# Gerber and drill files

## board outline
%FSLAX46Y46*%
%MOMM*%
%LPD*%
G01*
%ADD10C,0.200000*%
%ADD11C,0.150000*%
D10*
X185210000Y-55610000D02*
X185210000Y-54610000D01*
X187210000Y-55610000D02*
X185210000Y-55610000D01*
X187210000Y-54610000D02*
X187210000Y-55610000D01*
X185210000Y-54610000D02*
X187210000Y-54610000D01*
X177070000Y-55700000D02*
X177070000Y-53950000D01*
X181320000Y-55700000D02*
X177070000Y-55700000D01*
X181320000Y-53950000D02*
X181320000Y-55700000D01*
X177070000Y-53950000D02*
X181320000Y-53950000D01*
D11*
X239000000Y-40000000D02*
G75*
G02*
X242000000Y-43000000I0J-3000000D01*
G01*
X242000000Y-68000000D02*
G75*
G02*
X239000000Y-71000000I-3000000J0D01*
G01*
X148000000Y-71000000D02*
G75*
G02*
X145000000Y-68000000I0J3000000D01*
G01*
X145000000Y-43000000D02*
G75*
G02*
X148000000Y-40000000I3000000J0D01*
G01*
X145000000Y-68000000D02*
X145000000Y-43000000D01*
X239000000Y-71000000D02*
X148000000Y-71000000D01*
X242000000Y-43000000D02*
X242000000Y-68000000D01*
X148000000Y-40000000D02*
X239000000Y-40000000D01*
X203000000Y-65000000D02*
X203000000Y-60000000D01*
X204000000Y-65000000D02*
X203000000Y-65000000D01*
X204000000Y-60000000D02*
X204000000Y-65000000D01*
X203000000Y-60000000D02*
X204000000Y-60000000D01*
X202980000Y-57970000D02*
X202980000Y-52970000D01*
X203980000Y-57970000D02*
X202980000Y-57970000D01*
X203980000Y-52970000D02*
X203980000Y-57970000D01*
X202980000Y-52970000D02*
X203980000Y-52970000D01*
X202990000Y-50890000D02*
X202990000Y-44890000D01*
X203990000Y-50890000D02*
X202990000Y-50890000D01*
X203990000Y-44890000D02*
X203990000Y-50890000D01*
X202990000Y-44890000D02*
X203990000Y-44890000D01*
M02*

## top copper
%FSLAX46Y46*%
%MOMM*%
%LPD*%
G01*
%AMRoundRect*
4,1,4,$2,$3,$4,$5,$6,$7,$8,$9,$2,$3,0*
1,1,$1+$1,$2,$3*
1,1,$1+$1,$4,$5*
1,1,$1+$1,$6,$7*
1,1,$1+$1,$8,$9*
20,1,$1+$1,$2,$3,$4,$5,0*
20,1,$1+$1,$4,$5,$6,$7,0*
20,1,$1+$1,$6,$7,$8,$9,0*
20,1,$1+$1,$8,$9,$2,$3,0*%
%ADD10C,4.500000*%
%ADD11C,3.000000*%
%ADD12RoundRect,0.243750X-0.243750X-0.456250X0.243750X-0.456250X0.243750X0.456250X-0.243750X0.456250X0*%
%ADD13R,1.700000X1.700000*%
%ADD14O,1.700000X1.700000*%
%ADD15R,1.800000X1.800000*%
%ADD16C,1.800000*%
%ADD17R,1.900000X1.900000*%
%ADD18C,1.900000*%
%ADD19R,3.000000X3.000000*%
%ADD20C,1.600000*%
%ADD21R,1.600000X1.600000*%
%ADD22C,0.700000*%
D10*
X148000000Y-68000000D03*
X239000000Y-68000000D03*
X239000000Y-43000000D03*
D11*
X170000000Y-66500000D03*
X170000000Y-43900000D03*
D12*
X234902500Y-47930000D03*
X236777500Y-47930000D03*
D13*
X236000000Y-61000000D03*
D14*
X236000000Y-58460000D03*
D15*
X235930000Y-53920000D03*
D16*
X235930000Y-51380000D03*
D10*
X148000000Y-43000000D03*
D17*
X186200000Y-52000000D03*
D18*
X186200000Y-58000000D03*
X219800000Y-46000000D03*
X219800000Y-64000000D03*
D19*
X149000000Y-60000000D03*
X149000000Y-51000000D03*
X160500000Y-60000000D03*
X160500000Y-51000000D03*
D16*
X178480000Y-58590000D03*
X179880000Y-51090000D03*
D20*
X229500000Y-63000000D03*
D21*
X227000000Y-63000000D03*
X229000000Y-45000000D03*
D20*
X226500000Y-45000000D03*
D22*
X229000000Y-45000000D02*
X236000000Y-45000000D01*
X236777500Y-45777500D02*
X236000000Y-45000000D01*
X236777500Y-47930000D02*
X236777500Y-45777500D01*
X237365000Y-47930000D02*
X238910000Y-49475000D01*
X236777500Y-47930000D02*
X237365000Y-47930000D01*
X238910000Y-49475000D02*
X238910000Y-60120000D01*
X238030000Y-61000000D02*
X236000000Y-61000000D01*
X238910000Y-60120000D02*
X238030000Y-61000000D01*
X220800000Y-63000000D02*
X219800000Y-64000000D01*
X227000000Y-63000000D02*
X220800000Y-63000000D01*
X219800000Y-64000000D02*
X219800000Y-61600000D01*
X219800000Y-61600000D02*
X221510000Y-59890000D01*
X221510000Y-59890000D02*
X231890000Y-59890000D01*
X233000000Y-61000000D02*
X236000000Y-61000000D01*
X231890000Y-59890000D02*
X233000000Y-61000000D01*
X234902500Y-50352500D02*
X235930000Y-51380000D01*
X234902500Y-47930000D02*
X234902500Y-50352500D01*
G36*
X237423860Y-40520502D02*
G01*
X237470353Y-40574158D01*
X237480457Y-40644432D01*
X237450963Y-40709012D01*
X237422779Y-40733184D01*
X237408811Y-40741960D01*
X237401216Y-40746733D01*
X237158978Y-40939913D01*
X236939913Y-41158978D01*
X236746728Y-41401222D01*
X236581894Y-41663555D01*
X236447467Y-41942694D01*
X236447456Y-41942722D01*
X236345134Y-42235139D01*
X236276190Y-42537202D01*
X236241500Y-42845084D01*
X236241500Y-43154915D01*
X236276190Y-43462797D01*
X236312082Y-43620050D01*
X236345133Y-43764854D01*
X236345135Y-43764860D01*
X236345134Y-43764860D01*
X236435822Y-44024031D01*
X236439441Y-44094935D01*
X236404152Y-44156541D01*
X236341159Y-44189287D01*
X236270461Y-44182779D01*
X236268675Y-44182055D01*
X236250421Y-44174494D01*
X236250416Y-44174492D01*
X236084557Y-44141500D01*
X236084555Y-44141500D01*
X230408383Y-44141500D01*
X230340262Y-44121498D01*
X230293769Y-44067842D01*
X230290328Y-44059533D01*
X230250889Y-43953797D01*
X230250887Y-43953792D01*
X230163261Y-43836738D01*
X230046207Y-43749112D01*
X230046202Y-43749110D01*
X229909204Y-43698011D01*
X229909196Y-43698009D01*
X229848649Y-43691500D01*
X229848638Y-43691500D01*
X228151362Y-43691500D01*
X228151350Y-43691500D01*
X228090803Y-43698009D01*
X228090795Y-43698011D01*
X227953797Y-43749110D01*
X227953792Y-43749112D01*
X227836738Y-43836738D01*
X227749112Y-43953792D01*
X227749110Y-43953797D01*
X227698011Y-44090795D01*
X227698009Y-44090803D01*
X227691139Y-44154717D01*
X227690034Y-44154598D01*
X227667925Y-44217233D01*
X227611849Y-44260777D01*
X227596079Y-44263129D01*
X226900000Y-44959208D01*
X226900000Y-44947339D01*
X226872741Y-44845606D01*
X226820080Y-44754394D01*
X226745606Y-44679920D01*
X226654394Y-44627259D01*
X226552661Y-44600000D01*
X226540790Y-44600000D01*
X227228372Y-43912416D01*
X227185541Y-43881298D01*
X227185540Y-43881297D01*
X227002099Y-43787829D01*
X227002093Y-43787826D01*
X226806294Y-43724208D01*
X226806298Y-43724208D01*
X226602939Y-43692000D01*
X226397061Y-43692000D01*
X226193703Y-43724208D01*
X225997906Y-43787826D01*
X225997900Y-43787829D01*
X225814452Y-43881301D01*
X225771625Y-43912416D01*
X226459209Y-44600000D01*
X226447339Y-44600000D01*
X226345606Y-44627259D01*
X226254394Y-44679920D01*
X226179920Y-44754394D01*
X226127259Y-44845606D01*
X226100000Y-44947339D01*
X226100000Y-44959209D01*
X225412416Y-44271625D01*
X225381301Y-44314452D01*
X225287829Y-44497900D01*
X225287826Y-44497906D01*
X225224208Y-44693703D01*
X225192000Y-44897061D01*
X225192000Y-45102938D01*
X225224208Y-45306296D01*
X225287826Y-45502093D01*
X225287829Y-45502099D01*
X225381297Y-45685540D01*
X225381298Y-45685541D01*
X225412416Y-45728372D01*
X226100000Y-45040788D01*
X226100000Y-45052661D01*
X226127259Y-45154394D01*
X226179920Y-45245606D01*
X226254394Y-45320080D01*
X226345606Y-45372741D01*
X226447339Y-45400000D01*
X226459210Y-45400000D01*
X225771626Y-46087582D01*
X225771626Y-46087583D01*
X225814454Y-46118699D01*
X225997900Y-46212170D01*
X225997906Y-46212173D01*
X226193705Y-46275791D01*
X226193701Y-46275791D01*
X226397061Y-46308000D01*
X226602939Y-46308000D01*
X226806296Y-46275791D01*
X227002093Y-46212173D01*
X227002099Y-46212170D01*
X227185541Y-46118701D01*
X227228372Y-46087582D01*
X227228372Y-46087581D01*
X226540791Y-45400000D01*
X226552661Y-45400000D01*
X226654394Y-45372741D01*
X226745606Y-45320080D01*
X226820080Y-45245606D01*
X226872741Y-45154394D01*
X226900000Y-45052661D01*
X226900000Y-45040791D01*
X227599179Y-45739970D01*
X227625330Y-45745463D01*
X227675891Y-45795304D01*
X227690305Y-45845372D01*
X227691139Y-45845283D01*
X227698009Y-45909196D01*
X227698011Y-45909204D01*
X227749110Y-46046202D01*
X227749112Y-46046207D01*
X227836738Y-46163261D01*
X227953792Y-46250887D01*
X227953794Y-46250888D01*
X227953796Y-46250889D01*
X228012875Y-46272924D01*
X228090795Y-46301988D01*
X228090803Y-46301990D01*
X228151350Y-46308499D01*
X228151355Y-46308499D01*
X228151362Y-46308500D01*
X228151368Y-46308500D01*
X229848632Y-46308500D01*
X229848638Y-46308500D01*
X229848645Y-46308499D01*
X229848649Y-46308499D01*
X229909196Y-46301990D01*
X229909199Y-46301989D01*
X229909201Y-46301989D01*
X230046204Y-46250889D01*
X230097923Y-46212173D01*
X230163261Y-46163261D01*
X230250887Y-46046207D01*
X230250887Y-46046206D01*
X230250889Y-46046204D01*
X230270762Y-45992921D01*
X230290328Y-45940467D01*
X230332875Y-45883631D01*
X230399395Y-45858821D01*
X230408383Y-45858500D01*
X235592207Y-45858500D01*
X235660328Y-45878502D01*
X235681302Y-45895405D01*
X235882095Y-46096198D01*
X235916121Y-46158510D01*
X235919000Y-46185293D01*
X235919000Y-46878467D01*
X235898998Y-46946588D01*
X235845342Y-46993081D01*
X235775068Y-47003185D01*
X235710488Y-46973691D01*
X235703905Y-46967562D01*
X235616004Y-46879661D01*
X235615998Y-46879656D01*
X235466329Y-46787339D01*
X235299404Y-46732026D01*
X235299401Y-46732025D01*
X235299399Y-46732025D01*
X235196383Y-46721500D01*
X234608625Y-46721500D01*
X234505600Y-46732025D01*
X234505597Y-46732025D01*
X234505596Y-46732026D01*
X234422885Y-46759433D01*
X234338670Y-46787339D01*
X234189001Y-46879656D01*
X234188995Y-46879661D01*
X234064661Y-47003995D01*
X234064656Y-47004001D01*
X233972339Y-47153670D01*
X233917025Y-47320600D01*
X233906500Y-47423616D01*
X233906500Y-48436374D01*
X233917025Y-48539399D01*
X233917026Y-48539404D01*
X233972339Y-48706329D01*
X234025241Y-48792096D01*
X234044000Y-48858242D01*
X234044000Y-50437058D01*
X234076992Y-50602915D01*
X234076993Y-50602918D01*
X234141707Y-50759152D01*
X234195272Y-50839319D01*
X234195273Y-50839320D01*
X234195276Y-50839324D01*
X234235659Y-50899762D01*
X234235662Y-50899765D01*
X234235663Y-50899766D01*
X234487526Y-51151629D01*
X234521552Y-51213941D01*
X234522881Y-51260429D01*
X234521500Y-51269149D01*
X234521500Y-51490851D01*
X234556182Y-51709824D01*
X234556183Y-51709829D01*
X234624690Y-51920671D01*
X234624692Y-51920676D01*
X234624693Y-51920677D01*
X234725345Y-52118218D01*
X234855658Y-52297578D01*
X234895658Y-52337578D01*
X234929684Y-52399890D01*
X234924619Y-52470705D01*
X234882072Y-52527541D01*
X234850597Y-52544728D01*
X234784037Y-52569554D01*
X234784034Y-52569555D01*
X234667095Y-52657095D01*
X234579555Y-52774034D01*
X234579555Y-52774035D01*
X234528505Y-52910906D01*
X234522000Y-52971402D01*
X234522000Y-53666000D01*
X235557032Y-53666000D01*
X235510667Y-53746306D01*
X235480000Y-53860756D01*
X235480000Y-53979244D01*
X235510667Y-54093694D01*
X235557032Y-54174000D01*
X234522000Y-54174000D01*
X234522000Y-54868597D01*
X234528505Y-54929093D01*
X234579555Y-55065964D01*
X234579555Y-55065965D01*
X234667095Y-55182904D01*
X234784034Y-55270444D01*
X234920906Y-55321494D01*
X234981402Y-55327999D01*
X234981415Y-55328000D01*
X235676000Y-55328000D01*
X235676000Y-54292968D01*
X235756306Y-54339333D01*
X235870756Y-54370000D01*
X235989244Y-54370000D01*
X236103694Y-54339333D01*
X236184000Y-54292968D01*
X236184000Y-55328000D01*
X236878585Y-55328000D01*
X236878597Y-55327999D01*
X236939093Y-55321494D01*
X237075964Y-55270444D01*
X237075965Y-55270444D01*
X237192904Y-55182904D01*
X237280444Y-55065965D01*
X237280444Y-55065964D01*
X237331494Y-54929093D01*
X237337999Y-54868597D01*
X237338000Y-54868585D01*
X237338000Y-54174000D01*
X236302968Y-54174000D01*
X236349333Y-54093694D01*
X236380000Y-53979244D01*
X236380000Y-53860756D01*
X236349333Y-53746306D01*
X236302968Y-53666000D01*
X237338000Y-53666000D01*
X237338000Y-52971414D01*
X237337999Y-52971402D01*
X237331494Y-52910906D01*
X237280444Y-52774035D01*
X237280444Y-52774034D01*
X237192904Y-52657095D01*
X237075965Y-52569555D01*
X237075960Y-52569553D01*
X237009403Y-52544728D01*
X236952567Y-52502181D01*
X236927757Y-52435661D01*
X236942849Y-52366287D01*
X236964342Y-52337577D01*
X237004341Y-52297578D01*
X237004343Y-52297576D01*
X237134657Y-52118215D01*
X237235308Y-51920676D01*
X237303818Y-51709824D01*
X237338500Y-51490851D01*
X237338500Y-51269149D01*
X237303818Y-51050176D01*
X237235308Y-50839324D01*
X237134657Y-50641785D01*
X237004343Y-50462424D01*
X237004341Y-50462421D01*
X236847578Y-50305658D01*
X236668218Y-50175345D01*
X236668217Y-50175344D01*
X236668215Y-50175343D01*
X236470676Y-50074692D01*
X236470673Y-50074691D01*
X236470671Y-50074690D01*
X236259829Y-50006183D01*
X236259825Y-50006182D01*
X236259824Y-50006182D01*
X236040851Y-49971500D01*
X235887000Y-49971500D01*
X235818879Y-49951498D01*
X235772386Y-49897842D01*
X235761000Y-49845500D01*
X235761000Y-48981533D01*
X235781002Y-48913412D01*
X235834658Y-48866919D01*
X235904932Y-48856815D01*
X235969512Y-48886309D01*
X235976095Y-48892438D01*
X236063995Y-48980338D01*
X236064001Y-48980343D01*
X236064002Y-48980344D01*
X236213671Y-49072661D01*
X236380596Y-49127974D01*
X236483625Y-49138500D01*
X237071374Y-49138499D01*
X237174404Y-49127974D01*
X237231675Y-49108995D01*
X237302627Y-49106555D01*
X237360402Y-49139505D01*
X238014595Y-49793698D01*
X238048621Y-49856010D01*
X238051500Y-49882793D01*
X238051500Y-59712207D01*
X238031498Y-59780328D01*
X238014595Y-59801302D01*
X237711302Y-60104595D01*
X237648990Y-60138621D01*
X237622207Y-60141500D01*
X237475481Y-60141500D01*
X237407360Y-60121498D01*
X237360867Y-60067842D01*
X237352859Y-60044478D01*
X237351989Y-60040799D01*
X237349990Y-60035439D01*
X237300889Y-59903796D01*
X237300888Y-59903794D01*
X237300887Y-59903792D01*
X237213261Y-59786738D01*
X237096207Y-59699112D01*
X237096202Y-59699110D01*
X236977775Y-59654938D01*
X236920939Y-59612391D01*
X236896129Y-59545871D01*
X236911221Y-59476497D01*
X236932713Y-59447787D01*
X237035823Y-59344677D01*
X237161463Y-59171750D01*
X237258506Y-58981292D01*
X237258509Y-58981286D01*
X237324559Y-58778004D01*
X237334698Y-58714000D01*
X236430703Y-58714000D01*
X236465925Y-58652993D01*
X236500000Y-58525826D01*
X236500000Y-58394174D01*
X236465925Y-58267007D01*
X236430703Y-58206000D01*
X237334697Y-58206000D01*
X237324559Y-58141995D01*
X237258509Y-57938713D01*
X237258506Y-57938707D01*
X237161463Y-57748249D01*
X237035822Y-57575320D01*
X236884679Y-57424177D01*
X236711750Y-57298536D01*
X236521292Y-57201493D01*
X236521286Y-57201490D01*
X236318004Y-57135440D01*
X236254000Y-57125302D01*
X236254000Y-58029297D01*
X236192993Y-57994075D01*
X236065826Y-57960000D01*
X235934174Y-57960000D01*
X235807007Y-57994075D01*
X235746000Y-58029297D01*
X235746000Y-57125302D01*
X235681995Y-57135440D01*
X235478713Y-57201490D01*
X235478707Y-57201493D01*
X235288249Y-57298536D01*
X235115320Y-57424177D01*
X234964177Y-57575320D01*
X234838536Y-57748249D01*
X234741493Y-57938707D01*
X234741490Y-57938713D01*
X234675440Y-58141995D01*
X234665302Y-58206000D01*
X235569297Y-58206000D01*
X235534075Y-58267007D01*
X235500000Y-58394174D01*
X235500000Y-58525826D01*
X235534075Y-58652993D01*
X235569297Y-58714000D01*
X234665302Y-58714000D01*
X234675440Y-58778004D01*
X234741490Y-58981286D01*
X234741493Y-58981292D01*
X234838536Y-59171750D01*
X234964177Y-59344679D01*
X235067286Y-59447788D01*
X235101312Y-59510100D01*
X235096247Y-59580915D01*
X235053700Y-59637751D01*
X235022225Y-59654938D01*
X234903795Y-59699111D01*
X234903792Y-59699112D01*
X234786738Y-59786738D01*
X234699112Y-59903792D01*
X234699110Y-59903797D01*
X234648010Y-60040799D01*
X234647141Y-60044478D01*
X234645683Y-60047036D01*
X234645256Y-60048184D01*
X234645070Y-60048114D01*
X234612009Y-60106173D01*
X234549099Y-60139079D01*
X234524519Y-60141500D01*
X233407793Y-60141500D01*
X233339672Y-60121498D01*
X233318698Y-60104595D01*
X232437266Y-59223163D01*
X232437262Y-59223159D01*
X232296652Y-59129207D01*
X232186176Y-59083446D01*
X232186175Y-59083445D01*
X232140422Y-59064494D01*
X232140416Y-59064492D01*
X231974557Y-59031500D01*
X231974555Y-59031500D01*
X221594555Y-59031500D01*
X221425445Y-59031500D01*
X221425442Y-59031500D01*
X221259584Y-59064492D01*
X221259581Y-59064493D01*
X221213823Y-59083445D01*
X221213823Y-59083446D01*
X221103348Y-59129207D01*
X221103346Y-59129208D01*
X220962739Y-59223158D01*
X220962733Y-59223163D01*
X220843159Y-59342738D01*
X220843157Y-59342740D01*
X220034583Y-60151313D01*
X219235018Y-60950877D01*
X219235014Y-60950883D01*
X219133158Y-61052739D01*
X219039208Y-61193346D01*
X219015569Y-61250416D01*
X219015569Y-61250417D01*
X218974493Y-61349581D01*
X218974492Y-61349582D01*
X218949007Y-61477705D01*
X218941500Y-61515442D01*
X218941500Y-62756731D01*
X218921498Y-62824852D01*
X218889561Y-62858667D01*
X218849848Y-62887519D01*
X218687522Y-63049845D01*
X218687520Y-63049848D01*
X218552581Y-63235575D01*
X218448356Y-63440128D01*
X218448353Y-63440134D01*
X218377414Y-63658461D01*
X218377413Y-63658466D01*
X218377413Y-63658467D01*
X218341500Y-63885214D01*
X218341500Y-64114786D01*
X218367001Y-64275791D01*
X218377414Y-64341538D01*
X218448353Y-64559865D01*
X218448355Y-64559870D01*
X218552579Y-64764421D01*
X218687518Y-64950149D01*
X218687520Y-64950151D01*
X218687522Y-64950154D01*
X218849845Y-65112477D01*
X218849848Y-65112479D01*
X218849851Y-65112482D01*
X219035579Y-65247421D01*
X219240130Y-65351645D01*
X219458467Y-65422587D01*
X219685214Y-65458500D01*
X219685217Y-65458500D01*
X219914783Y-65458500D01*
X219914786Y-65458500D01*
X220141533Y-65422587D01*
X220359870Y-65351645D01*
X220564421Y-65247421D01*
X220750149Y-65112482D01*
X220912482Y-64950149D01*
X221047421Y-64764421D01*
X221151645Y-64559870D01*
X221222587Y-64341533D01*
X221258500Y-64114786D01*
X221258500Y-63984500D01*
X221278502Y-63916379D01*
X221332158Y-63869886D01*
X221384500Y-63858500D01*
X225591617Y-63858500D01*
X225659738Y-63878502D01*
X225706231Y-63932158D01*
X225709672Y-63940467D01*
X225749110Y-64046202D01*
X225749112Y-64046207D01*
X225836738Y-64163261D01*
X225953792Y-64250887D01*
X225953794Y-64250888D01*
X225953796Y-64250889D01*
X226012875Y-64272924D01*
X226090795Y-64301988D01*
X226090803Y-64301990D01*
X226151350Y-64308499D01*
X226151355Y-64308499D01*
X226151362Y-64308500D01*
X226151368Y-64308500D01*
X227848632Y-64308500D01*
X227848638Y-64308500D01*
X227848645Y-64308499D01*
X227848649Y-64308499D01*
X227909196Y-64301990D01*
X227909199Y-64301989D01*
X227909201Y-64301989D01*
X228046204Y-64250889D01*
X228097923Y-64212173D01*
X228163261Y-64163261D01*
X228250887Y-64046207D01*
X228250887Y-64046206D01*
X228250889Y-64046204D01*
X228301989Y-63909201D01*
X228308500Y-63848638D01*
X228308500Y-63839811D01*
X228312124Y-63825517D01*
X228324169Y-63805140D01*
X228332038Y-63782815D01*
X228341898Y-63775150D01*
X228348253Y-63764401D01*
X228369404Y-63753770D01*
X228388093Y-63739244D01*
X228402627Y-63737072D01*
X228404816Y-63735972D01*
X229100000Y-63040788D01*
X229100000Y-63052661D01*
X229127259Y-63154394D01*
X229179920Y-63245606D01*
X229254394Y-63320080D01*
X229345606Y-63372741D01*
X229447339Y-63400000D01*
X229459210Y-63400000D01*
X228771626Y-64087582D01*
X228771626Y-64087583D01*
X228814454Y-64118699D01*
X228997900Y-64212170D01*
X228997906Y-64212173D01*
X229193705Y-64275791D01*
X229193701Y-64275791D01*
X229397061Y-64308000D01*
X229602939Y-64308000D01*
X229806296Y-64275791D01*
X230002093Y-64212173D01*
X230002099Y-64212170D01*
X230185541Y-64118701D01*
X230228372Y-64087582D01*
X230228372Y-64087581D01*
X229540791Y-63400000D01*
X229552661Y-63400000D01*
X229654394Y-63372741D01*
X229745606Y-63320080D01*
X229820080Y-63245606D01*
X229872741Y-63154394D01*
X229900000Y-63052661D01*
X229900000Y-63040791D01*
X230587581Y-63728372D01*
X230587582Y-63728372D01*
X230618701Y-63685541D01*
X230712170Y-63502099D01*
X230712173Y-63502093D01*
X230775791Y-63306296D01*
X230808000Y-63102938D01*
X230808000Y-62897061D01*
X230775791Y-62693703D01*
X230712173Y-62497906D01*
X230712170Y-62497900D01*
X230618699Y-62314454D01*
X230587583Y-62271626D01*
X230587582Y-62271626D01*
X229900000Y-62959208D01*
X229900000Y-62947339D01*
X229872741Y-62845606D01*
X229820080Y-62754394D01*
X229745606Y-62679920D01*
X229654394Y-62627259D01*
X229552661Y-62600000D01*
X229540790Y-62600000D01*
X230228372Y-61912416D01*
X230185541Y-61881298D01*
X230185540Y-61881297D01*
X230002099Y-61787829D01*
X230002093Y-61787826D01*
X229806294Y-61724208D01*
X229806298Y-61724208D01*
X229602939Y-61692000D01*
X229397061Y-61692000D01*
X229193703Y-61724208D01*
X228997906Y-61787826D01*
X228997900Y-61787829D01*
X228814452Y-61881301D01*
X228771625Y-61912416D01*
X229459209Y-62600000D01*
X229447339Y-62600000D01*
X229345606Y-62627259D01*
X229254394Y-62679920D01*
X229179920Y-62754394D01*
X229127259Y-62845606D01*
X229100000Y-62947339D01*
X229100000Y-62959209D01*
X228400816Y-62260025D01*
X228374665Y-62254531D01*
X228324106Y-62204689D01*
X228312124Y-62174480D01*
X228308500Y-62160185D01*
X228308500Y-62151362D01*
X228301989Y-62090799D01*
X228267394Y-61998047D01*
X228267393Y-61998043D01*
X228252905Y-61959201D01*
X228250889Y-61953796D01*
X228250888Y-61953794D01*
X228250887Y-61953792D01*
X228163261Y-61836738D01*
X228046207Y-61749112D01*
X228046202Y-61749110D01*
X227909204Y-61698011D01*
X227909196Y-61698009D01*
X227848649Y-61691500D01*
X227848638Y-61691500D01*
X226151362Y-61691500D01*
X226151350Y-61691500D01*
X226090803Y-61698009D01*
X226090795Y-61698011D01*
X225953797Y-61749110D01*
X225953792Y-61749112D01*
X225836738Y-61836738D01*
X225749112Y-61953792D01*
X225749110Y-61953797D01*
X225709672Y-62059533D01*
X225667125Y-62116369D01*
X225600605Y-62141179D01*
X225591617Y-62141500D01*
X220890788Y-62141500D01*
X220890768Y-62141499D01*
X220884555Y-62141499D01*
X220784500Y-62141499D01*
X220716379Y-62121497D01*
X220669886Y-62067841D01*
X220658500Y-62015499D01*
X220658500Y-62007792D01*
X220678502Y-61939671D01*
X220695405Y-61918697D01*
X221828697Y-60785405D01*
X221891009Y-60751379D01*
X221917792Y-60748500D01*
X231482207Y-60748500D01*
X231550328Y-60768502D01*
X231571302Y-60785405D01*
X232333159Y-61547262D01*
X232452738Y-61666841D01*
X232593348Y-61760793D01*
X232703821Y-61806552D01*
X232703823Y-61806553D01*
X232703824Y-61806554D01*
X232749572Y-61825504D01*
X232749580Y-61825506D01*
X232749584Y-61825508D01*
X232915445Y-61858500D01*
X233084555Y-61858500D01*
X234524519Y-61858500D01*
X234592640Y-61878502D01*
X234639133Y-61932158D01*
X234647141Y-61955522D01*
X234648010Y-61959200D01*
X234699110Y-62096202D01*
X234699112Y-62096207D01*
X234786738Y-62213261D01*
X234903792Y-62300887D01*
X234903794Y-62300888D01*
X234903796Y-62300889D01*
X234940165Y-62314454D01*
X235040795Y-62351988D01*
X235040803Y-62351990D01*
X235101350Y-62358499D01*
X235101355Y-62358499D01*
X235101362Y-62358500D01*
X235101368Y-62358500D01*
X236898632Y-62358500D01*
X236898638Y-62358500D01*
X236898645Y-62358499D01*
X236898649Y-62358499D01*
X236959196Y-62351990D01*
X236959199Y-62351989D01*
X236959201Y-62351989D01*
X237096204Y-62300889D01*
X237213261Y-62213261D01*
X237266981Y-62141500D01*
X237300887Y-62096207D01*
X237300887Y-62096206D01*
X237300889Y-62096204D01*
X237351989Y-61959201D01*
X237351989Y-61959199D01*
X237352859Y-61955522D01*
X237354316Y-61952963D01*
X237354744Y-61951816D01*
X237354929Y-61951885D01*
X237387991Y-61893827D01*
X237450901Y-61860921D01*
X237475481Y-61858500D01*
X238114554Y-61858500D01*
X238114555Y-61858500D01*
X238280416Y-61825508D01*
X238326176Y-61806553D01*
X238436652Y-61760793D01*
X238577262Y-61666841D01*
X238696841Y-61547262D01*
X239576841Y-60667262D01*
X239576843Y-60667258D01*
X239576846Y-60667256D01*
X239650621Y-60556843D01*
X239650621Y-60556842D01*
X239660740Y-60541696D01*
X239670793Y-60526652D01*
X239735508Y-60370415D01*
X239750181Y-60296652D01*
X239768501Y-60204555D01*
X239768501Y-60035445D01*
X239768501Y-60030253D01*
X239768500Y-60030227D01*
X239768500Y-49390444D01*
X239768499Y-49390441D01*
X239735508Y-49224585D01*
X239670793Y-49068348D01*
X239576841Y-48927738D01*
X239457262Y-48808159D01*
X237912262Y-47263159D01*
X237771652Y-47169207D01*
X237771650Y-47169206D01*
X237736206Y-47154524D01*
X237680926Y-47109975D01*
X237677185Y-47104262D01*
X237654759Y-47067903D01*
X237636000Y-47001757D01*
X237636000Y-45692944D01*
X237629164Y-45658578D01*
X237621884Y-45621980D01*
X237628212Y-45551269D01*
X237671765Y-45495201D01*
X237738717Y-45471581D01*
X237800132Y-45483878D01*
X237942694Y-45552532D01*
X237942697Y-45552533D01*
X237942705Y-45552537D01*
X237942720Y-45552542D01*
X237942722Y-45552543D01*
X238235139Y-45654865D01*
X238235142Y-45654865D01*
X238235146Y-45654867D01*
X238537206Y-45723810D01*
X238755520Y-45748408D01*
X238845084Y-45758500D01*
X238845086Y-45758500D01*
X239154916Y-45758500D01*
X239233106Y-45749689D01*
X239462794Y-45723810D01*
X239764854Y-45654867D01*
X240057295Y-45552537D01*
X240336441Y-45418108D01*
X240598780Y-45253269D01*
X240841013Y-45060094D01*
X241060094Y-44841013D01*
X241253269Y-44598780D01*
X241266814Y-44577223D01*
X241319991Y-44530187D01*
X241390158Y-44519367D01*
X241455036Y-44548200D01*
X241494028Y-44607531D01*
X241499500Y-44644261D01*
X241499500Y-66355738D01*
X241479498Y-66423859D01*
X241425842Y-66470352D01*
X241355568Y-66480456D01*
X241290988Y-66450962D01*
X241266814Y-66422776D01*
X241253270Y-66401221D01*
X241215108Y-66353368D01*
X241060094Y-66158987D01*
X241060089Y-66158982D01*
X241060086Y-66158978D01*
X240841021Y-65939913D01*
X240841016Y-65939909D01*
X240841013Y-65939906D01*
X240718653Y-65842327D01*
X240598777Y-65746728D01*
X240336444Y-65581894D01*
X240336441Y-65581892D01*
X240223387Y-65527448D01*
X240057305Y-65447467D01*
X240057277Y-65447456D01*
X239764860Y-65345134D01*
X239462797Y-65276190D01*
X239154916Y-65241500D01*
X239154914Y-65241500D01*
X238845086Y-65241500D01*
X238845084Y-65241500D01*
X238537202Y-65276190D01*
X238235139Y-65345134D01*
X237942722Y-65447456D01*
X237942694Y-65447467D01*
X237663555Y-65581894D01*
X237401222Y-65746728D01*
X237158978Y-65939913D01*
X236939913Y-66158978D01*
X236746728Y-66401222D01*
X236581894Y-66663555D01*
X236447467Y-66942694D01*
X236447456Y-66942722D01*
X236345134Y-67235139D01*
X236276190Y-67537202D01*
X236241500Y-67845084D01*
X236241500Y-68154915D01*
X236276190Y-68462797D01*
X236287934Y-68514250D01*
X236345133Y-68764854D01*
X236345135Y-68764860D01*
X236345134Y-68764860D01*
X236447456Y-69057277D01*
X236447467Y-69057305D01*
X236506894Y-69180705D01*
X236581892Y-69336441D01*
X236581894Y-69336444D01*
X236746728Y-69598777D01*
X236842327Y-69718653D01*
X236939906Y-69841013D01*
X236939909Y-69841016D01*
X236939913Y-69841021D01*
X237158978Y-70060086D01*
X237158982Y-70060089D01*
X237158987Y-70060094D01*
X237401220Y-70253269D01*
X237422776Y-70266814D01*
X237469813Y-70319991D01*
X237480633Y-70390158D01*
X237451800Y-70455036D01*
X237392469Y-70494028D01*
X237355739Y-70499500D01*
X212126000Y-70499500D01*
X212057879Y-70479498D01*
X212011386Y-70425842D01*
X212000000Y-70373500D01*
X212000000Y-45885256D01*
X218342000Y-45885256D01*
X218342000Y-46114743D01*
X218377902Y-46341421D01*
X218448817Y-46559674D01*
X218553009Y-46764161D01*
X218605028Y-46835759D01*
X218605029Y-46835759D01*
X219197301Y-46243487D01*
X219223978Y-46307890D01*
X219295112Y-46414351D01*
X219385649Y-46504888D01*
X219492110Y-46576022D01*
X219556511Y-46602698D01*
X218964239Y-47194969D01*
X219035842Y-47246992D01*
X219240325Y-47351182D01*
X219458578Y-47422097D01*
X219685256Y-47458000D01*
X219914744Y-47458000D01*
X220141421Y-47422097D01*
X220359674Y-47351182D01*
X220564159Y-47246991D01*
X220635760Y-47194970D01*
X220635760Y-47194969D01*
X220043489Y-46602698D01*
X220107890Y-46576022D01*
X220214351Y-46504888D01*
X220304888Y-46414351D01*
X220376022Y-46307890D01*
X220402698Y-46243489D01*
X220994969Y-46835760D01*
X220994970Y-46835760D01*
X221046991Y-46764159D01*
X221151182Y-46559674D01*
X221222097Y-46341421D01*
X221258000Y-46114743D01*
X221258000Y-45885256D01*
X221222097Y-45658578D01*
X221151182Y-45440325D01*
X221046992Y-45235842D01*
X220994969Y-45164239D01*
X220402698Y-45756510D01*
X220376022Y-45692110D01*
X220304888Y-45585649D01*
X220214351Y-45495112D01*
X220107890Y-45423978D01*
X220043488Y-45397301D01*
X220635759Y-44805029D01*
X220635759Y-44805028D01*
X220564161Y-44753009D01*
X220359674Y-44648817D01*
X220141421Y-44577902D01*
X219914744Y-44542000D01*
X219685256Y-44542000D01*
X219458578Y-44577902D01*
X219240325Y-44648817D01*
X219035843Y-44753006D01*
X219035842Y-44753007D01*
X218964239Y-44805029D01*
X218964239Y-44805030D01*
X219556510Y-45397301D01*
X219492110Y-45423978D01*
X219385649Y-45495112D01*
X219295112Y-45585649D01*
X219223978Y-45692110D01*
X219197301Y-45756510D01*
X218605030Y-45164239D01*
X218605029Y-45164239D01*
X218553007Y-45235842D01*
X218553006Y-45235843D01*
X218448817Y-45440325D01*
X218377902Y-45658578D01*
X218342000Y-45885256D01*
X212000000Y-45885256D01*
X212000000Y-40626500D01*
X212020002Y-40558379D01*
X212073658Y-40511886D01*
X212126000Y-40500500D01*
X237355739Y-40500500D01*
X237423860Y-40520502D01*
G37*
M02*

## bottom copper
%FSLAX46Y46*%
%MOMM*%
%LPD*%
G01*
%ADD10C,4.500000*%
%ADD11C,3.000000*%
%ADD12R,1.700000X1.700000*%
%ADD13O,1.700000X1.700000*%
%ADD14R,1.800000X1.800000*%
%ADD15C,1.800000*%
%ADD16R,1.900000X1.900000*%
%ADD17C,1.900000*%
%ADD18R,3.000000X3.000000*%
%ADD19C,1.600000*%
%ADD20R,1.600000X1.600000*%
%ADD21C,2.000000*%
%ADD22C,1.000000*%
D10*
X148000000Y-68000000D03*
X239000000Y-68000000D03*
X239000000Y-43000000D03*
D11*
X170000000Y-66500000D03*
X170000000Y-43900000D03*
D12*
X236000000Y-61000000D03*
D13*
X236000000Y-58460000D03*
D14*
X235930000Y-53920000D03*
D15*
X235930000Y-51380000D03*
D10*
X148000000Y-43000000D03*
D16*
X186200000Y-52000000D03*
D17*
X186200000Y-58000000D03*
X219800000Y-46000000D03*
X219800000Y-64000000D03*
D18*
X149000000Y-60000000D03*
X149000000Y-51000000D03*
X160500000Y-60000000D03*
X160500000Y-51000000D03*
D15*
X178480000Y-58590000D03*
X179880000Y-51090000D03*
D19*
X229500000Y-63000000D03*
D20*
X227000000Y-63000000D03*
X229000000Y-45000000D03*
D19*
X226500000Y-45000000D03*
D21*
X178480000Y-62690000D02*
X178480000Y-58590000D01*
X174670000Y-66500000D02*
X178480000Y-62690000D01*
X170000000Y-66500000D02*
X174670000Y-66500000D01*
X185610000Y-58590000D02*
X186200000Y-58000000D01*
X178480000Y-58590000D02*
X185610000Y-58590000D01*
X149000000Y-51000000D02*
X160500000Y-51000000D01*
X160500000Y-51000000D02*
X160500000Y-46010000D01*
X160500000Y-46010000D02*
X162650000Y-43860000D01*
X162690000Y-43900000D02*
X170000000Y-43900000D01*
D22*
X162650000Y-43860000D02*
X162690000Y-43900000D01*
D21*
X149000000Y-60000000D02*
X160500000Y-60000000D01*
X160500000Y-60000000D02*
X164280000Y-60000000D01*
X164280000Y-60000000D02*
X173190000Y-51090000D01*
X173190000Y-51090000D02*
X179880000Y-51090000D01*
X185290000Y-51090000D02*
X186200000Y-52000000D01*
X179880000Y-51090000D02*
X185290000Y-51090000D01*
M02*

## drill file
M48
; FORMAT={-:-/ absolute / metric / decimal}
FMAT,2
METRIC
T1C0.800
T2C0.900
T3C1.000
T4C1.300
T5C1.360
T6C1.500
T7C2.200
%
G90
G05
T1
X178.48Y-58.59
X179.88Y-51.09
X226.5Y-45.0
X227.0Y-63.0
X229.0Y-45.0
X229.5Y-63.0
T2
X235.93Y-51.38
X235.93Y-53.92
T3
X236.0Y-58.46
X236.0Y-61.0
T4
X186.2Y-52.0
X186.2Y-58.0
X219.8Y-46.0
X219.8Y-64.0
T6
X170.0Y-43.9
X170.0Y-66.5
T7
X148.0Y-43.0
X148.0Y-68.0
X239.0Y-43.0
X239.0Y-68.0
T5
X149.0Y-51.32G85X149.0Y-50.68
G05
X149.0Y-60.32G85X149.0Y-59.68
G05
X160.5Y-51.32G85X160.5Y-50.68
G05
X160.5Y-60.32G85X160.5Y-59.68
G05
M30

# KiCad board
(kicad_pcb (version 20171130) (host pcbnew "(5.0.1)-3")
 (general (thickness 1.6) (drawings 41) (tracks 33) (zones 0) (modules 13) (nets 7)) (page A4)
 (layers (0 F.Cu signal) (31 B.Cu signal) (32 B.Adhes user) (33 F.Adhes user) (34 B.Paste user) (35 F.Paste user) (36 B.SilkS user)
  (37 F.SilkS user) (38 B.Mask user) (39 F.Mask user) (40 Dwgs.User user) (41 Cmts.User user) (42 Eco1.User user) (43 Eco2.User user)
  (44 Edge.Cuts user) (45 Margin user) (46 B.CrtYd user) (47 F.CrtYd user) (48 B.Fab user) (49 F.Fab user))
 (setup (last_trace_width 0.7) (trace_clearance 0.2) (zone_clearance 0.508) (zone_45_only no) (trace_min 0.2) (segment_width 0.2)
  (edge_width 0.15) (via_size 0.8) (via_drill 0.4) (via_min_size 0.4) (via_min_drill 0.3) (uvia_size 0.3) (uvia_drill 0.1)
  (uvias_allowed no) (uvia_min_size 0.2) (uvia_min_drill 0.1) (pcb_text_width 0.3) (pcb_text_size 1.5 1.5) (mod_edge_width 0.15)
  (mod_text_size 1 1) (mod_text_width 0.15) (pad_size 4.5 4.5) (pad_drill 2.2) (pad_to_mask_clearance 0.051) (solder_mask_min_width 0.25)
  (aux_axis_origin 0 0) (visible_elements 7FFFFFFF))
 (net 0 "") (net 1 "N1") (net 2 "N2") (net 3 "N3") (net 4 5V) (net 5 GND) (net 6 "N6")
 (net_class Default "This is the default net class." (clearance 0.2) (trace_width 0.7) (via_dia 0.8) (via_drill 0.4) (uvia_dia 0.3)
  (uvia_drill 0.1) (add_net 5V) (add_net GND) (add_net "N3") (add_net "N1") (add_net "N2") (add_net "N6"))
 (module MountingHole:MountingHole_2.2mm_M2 (layer F.Cu) (at 148 68)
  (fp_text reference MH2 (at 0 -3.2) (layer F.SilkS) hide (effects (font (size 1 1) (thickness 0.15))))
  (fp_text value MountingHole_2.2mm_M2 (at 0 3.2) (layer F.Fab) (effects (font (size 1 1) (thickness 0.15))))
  (pad "" np_thru_hole circle (at 0 0) (size 4.5 4.5) (drill 2.2) (layers *.Cu *.Mask)))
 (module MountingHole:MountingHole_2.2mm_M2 (layer F.Cu) (at 239 68)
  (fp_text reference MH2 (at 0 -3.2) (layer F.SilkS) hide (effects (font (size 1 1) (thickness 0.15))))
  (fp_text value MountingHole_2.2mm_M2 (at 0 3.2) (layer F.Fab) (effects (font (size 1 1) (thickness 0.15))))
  (pad "" np_thru_hole circle (at 0 0) (size 4.5 4.5) (drill 2.2) (layers *.Cu *.Mask)))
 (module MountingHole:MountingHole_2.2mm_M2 (layer F.Cu) (at 239 43)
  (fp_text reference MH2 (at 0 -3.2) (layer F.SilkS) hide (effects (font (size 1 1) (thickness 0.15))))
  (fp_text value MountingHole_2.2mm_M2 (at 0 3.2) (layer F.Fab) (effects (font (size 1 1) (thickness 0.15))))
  (pad "" np_thru_hole circle (at 0 0) (size 4.5 4.5) (drill 2.2) (layers *.Cu *.Mask)))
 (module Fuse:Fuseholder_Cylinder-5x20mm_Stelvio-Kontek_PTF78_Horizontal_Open (layer F.Cu) (at 170 66.5 90)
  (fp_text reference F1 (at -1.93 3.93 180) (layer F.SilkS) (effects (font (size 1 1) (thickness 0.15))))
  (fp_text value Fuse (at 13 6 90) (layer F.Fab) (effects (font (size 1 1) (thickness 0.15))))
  (pad 1 thru_hole circle (at 0 0 90) (size 3 3) (drill 1.5) (layers *.Cu *.Mask) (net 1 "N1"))
  (pad 2 thru_hole circle (at 22.6 0 90) (size 3 3) (drill 1.5) (layers *.Cu *.Mask) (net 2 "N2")))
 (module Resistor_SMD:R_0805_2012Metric (layer F.Cu) (at 235.84 47.93)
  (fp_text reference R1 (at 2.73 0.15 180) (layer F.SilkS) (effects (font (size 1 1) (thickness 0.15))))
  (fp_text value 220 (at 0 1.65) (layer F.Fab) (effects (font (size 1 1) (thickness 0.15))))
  (pad 1 smd roundrect (at -0.9375 0) (size 0.975 1.4) (layers F.Cu F.Paste F.Mask) (roundrect_rratio 0.25) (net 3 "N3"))
  (pad 2 smd roundrect (at 0.9375 0) (size 0.975 1.4) (layers F.Cu F.Paste F.Mask) (roundrect_rratio 0.25) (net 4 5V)))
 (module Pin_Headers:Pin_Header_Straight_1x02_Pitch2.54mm (layer F.Cu) (at 236 61 180)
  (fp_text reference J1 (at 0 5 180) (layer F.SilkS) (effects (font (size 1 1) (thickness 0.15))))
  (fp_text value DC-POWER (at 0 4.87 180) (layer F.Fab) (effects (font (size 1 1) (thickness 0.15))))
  (pad 1 thru_hole rect (at 0 0 180) (size 1.7 1.7) (drill 1) (layers *.Cu *.Mask) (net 4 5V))
  (pad 2 thru_hole oval (at 0 2.54 180) (size 1.7 1.7) (drill 1) (layers *.Cu *.Mask) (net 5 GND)))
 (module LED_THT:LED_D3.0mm (layer F.Cu) (at 235.93 53.92 90)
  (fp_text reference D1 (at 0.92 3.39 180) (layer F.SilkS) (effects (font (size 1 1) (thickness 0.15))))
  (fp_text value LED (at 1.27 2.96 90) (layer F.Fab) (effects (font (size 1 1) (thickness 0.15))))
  (pad 1 thru_hole rect (at 0 0 90) (size 1.8 1.8) (drill 0.9) (layers *.Cu *.Mask) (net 5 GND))
  (pad 2 thru_hole circle (at 2.54 0 90) (size 1.8 1.8) (drill 0.9) (layers *.Cu *.Mask) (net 3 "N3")))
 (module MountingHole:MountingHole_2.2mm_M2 (layer F.Cu) (at 148 43)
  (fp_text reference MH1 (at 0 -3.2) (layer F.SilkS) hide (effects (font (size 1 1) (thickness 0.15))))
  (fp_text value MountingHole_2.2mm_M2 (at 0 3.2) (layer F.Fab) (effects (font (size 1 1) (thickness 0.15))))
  (pad "" np_thru_hole circle (at 0 0) (size 4.5 4.5) (drill 2.2) (layers *.Cu *.Mask)))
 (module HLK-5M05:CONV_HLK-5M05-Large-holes (layer F.Cu) (at 203 55)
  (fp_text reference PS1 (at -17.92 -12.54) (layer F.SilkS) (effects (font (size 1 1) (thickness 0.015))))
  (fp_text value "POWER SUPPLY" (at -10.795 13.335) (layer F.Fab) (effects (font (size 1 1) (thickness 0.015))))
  (pad 1 thru_hole rect (at -16.8 -3) (size 1.9 1.9) (drill 1.3) (layers *.Cu *.Mask) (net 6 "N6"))
  (pad 2 thru_hole circle (at -16.8 3) (size 1.9 1.9) (drill 1.3) (layers *.Cu *.Mask) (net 1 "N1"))
  (pad 3 thru_hole circle (at 16.8 -9) (size 1.9 1.9) (drill 1.3) (layers *.Cu *.Mask) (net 5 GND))
  (pad 4 thru_hole circle (at 16.8 9) (size 1.9 1.9) (drill 1.3) (layers *.Cu *.Mask) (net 4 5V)))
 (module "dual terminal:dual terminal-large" (layer F.Cu) (at 149 60 90)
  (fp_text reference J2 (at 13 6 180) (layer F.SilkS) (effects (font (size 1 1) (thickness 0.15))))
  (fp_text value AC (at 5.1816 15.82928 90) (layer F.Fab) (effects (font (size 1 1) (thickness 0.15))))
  (pad 1 thru_hole rect (at 0 0 90) (size 3 3) (drill oval 2 1.36) (layers *.Cu *.Mask) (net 6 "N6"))
  (pad 2 thru_hole rect (at 9 0 90) (size 3 3) (drill oval 2 1.36) (layers *.Cu *.Mask) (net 2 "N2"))
  (pad 1 thru_hole rect (at 0 11.5 90) (size 3 3) (drill oval 2 1.36) (layers *.Cu *.Mask) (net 6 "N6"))
  (pad 2 thru_hole rect (at 9 11.5 90) (size 3 3) (drill oval 2 1.36) (layers *.Cu *.Mask) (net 2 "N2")))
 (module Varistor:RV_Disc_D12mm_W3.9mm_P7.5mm (layer F.Cu) (at 178.48 58.59 90)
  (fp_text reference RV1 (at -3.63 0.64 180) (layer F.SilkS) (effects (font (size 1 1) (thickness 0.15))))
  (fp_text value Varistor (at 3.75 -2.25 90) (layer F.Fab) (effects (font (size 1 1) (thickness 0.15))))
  (pad 1 thru_hole circle (at 0 0 90) (size 1.8 1.8) (drill 0.8) (layers *.Cu *.Mask) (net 1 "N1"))
  (pad 2 thru_hole circle (at 7.5 1.4 90) (size 1.8 1.8) (drill 0.8) (layers *.Cu *.Mask) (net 6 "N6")))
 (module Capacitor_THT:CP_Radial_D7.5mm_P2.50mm (layer F.Cu) (at 227 63)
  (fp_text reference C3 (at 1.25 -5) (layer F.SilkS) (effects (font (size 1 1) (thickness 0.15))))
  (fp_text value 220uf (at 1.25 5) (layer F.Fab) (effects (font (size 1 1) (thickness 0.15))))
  (pad 2 thru_hole circle (at 2.5 0) (size 1.6 1.6) (drill 0.8) (layers *.Cu *.Mask) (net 5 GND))
  (pad 1 thru_hole rect (at 0 0) (size 1.6 1.6) (drill 0.8) (layers *.Cu *.Mask) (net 4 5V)))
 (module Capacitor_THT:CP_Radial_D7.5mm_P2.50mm (layer F.Cu) (at 229 45 180)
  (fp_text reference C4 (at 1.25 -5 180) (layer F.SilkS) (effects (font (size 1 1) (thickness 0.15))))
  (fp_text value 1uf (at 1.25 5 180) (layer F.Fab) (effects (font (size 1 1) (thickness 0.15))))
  (pad 1 thru_hole rect (at 0 0 180) (size 1.6 1.6) (drill 0.8) (layers *.Cu *.Mask) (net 4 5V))
  (pad 2 thru_hole circle (at 2.5 0 180) (size 1.6 1.6) (drill 0.8) (layers *.Cu *.Mask) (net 5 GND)))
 (gr_line (start 185.21 55.61) (end 185.21 54.61) (layer Edge.Cuts) (width 0.2))
 (gr_line (start 187.21 55.61) (end 185.21 55.61) (layer Edge.Cuts) (width 0.2))
 (gr_line (start 187.21 54.61) (end 187.21 55.61) (layer Edge.Cuts) (width 0.2))
 (gr_line (start 185.21 54.61) (end 187.21 54.61) (layer Edge.Cuts) (width 0.2))
 (gr_line (start 177.07 55.7) (end 177.07 53.95) (layer Edge.Cuts) (width 0.2))
 (gr_line (start 181.32 55.7) (end 177.07 55.7) (layer Edge.Cuts) (width 0.2))
 (gr_line (start 181.32 53.95) (end 181.32 55.7) (layer Edge.Cuts) (width 0.2))
 (gr_line (start 177.07 53.95) (end 181.32 53.95) (layer Edge.Cuts) (width 0.2))
 (gr_arc (start 239 43) (end 242 43) (angle -90) (layer Edge.Cuts) (width 0.15))
 (gr_arc (start 239 68) (end 239 71) (angle -90) (layer Edge.Cuts) (width 0.15))
 (gr_arc (start 148 68) (end 145 68) (angle -90) (layer Edge.Cuts) (width 0.15))
 (gr_arc (start 148 43) (end 148 40) (angle -90) (layer Edge.Cuts) (width 0.15))
 (gr_line (start 145 68) (end 145 43) (layer Edge.Cuts) (width 0.15))
 (gr_line (start 239 71) (end 148 71) (layer Edge.Cuts) (width 0.15))
 (gr_line (start 242 43) (end 242 68) (layer Edge.Cuts) (width 0.15))
 (gr_line (start 148 40) (end 239 40) (layer Edge.Cuts) (width 0.15))
 (gr_line (start 203 65) (end 203 60) (layer Edge.Cuts) (width 0.15))
 (gr_line (start 204 65) (end 203 65) (layer Edge.Cuts) (width 0.15))
 (gr_line (start 204 60) (end 204 65) (layer Edge.Cuts) (width 0.15))
 (gr_line (start 203 60) (end 204 60) (layer Edge.Cuts) (width 0.15))
 (gr_line (start 202.98 57.97) (end 202.98 52.97) (layer Edge.Cuts) (width 0.15))
 (gr_line (start 203.98 57.97) (end 202.98 57.97) (layer Edge.Cuts) (width 0.15))
 (gr_line (start 203.98 52.97) (end 203.98 57.97) (layer Edge.Cuts) (width 0.15))
 (gr_line (start 202.98 52.97) (end 203.98 52.97) (layer Edge.Cuts) (width 0.15))
 (gr_line (start 202.99 50.89) (end 202.99 44.89) (layer Edge.Cuts) (width 0.15))
 (gr_line (start 203.99 50.89) (end 202.99 50.89) (layer Edge.Cuts) (width 0.15))
 (gr_line (start 203.99 44.89) (end 203.99 50.89) (layer Edge.Cuts) (width 0.15))
 (gr_line (start 202.99 44.89) (end 203.99 44.89) (layer Edge.Cuts) (width 0.15))
 (segment (start 178.48 62.69) (end 178.48 58.59) (width 2) (layer B.Cu) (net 1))
 (segment (start 174.67 66.5) (end 178.48 62.69) (width 2) (layer B.Cu) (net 1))
 (segment (start 170 66.5) (end 174.67 66.5) (width 2) (layer B.Cu) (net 1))
 (segment (start 185.61 58.59) (end 186.2 58) (width 2) (layer B.Cu) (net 1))
 (segment (start 178.48 58.59) (end 185.61 58.59) (width 2) (layer B.Cu) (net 1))
 (segment (start 149 51) (end 160.5 51) (width 2) (layer B.Cu) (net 2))
 (segment (start 160.5 51) (end 160.5 46.01) (width 2) (layer B.Cu) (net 2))
 (segment (start 160.5 46.01) (end 162.65 43.86) (width 2) (layer B.Cu) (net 2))
 (segment (start 162.69 43.9) (end 170 43.9) (width 2) (layer B.Cu) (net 2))
 (segment (start 162.65 43.86) (end 162.69 43.9) (width 1) (layer B.Cu) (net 2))
 (segment (start 149 60) (end 160.5 60) (width 2) (layer B.Cu) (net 6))
 (segment (start 160.5 60) (end 164.28 60) (width 2) (layer B.Cu) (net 6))
 (segment (start 164.28 60) (end 173.19 51.09) (width 2) (layer B.Cu) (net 6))
 (segment (start 173.19 51.09) (end 179.88 51.09) (width 2) (layer B.Cu) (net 6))
 (segment (start 185.29 51.09) (end 186.2 52) (width 2) (layer B.Cu) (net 6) (status 1000000))
 (segment (start 179.88 51.09) (end 185.29 51.09) (width 2) (layer B.Cu) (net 6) (status 1000000))
 (segment (start 229 45) (end 236 45) (width 0.7) (layer F.Cu) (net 4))
 (segment (start 236.7775 45.7775) (end 236 45) (width 0.7) (layer F.Cu) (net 4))
 (segment (start 236.7775 47.93) (end 236.7775 45.7775) (width 0.7) (layer F.Cu) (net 4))
 (segment (start 237.365 47.93) (end 238.91 49.475) (width 0.7) (layer F.Cu) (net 4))
 (segment (start 236.7775 47.93) (end 237.365 47.93) (width 0.7) (layer F.Cu) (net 4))
 (segment (start 238.91 49.475) (end 238.91 60.12) (width 0.7) (layer F.Cu) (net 4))
 (segment (start 238.03 61) (end 236 61) (width 0.7) (layer F.Cu) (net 4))
 (segment (start 238.91 60.12) (end 238.03 61) (width 0.7) (layer F.Cu) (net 4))
 (segment (start 220.8 63) (end 219.8 64) (width 0.7) (layer F.Cu) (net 4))
 (segment (start 227 63) (end 220.8 63) (width 0.7) (layer F.Cu) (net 4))
 (segment (start 219.8 64) (end 219.8 61.6) (width 0.7) (layer F.Cu) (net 4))
 (segment (start 219.8 61.6) (end 221.51 59.89) (width 0.7) (layer F.Cu) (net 4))
 (segment (start 221.51 59.89) (end 231.89 59.89) (width 0.7) (layer F.Cu) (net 4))
 (segment (start 233 61) (end 236 61) (width 0.7) (layer F.Cu) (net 4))
 (segment (start 231.89 59.89) (end 233 61) (width 0.7) (layer F.Cu) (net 4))
 (segment (start 234.9025 50.3525) (end 235.93 51.38) (width 0.7) (layer F.Cu) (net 3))
 (segment (start 234.9025 47.93) (end 234.9025 50.3525) (width 0.7) (layer F.Cu) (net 3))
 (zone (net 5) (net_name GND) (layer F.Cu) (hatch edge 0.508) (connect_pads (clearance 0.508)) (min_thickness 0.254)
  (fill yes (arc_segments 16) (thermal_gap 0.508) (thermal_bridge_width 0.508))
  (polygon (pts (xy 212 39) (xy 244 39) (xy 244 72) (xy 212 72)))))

